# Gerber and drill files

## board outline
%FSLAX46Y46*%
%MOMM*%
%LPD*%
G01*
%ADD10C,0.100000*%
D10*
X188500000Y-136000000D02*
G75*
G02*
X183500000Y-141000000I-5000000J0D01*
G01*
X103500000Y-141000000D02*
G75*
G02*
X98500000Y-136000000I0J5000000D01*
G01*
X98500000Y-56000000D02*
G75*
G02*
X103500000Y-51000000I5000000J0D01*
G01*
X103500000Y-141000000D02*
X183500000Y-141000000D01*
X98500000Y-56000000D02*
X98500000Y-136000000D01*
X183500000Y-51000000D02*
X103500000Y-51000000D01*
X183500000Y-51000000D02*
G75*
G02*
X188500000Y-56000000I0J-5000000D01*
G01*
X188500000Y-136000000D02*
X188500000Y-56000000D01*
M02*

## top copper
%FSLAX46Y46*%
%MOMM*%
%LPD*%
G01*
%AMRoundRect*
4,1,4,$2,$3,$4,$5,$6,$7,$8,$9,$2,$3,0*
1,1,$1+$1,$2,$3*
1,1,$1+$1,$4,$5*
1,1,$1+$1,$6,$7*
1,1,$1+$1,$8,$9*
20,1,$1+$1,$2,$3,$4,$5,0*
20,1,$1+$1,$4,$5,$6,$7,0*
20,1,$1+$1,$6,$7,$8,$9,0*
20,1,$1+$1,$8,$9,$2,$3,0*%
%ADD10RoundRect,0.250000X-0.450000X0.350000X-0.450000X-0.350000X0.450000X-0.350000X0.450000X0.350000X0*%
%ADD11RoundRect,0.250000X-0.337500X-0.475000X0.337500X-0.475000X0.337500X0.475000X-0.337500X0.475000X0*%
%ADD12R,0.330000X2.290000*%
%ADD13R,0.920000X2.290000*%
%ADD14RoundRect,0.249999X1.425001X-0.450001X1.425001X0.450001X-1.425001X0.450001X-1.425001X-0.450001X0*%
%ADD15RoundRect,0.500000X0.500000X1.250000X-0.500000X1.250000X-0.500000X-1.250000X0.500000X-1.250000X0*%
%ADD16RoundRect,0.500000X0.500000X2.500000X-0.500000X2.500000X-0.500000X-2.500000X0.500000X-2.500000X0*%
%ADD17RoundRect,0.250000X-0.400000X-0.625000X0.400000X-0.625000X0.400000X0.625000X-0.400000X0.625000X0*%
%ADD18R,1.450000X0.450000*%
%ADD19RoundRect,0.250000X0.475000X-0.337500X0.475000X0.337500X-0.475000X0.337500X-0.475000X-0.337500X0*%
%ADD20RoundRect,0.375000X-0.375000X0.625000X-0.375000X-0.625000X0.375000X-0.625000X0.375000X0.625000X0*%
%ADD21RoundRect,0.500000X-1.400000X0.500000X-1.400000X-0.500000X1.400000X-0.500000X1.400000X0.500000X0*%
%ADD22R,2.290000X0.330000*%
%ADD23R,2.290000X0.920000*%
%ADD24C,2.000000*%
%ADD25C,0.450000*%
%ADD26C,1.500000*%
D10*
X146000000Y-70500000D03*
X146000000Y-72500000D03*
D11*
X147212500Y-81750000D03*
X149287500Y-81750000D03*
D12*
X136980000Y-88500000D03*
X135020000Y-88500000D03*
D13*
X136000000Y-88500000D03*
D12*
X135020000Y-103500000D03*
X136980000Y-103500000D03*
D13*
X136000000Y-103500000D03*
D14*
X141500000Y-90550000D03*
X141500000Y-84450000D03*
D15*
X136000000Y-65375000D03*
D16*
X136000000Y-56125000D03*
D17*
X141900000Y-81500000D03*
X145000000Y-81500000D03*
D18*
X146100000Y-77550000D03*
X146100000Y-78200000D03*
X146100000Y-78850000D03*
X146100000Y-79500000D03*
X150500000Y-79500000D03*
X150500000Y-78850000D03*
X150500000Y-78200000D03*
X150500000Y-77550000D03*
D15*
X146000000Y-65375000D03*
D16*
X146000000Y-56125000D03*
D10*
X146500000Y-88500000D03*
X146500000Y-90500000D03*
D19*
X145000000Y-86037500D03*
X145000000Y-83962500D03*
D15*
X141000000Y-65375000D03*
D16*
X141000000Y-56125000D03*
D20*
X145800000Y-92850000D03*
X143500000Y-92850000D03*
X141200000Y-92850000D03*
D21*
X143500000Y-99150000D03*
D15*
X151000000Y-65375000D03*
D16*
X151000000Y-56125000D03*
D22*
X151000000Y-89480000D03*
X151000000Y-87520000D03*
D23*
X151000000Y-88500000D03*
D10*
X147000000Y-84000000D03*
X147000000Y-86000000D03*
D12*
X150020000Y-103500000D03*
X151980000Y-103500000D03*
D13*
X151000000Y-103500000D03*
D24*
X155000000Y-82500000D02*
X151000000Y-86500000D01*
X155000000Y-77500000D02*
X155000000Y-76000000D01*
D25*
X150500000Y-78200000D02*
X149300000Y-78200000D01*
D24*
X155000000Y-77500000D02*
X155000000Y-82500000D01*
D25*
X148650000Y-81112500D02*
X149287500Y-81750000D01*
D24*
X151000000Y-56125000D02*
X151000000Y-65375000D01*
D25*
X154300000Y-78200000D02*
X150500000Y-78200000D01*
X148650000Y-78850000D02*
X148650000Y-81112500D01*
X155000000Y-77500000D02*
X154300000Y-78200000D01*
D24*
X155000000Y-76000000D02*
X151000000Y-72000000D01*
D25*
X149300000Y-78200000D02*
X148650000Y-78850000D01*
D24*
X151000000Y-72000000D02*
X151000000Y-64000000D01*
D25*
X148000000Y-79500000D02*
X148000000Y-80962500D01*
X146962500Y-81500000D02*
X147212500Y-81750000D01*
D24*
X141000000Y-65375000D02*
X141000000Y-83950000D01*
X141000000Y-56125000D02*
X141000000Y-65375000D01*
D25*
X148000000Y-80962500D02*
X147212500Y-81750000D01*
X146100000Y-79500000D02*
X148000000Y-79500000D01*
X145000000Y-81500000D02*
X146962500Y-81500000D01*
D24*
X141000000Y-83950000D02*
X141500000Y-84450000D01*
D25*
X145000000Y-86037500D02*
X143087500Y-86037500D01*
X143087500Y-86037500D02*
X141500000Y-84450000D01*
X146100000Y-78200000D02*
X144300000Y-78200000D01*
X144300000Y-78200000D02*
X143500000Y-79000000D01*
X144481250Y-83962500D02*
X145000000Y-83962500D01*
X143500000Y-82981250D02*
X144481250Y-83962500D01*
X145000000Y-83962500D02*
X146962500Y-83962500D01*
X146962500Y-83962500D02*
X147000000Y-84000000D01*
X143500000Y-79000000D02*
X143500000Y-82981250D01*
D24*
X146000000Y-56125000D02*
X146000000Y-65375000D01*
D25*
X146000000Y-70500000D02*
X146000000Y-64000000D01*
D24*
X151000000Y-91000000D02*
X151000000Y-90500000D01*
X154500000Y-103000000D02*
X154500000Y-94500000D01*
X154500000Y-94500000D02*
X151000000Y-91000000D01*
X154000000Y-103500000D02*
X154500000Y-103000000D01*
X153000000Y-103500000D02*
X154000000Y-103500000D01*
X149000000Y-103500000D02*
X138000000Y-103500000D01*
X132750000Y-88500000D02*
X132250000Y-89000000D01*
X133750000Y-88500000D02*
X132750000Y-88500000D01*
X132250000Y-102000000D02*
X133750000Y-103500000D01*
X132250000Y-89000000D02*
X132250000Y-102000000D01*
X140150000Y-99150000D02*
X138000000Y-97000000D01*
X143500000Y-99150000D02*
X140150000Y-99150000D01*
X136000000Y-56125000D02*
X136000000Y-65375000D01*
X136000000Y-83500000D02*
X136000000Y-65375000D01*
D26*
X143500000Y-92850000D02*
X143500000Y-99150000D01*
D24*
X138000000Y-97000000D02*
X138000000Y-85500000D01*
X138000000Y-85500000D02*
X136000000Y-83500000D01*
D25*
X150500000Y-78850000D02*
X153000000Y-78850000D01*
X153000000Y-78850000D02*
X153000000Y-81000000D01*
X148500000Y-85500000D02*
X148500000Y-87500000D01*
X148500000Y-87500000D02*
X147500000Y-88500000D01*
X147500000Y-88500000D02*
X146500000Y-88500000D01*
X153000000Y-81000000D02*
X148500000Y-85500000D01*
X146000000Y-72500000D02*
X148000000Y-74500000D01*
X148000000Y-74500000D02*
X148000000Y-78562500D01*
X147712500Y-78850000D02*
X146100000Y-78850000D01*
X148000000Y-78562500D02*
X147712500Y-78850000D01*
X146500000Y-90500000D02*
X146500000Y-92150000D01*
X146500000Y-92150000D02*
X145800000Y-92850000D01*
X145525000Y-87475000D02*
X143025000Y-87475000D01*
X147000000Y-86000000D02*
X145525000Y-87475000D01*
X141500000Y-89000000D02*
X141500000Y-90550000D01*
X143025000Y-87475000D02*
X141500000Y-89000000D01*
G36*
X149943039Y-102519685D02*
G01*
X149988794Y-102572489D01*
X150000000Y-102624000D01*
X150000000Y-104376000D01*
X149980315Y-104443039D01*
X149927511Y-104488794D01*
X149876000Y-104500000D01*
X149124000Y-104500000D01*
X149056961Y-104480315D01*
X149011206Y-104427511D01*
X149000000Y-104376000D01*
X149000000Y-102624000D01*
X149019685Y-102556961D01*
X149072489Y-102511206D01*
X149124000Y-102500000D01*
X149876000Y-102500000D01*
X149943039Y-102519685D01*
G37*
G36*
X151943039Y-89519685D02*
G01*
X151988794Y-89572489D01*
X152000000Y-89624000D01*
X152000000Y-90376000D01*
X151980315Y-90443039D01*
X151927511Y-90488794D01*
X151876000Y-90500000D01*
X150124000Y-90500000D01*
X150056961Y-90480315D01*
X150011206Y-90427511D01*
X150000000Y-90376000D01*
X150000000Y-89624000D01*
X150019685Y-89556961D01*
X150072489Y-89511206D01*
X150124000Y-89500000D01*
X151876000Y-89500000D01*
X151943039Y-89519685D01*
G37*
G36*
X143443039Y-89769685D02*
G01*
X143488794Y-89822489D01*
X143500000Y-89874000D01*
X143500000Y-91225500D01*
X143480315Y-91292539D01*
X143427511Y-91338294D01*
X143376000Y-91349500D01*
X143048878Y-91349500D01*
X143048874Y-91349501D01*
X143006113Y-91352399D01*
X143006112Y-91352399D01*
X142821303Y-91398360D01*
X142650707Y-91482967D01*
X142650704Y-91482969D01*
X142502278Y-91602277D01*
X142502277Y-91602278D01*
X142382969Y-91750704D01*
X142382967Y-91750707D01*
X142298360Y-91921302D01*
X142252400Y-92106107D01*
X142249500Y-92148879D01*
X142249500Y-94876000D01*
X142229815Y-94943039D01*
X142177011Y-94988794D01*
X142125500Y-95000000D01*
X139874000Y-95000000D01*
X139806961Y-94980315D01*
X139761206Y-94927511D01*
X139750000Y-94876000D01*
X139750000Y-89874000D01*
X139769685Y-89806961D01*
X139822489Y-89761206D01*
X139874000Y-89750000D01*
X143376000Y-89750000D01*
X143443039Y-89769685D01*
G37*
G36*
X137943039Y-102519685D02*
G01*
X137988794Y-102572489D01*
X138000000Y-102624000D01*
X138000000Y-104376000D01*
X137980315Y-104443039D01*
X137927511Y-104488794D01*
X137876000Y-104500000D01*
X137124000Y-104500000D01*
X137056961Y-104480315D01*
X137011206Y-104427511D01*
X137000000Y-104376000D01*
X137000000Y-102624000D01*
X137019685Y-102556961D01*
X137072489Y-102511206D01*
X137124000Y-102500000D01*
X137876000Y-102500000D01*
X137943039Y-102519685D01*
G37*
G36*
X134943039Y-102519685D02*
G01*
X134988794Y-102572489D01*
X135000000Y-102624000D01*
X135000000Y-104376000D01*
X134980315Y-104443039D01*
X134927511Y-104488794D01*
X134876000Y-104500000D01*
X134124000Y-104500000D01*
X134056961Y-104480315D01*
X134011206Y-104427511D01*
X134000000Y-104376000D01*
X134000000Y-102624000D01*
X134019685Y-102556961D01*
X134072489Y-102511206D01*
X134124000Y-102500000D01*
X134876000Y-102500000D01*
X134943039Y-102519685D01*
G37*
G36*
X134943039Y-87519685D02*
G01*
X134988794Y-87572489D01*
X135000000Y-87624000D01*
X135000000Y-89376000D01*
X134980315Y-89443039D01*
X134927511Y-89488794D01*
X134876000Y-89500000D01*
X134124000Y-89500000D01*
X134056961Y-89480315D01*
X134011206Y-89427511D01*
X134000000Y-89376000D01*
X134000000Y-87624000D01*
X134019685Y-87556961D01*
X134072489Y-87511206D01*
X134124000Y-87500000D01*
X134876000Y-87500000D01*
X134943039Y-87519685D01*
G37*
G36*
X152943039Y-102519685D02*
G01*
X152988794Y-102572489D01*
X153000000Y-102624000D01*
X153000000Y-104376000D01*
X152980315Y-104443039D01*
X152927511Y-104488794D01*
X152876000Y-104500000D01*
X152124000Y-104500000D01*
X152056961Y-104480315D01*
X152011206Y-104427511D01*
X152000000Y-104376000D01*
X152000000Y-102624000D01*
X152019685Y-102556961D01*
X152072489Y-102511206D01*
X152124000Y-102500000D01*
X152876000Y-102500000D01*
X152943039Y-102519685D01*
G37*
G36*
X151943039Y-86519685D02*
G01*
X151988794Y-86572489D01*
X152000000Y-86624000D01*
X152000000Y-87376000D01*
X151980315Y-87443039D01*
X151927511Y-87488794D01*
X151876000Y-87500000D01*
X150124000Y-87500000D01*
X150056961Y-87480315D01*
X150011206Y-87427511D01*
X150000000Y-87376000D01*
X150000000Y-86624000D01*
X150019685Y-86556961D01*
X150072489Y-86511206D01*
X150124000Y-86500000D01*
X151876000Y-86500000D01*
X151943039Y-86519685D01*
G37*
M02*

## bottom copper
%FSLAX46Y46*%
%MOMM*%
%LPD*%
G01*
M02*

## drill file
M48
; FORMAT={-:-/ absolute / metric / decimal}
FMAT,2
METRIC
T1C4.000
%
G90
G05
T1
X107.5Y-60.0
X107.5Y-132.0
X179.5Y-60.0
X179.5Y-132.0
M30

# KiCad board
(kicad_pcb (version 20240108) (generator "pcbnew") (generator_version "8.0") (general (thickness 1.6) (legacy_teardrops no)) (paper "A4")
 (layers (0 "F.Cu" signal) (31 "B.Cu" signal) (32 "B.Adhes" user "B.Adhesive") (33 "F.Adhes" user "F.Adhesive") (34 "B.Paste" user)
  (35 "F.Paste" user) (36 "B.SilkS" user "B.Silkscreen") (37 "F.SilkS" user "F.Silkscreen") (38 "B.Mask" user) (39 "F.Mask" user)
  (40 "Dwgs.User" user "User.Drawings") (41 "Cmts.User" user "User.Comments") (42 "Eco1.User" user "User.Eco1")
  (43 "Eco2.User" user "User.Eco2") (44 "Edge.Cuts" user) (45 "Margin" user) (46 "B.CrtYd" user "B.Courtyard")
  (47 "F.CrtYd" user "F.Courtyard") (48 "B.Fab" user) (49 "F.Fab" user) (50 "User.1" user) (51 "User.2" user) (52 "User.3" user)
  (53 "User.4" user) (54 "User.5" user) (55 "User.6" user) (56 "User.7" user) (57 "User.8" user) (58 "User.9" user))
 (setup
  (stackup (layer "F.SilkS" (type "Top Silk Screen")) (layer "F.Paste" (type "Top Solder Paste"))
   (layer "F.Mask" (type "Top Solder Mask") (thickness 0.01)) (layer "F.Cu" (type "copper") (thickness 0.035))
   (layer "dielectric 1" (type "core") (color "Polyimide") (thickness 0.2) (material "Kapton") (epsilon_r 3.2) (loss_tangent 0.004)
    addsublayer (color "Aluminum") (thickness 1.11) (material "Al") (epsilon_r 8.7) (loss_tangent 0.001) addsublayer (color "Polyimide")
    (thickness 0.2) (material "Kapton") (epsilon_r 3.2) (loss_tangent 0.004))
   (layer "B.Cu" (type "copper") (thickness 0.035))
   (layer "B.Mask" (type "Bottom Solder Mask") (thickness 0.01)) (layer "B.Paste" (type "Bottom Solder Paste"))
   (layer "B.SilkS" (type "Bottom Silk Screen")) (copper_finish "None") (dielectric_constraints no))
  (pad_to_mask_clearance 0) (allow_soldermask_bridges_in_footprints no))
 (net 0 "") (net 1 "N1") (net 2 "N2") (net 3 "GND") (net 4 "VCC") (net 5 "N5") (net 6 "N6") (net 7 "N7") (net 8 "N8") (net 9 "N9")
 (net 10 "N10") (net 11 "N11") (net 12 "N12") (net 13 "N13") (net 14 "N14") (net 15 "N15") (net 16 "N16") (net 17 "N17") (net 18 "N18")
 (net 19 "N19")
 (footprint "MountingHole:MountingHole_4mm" (layer "F.Cu") (at 179.5 132)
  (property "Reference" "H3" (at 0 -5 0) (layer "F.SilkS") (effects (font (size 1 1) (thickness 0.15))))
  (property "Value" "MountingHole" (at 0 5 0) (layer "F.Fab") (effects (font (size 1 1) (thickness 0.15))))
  (pad "" np_thru_hole circle (at 0 0) (size 4 4) (drill 4) (layers "*.Cu" "*.Mask")))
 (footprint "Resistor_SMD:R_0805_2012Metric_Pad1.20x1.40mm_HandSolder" (layer "F.Cu") (at 146 71.5 -90)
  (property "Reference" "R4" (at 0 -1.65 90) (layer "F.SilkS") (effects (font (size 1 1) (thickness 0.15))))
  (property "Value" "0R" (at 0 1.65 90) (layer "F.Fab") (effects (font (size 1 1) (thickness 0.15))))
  (pad "1" smd roundrect (at -1 0 270) (size 1.2 1.4) (layers "F.Cu" "F.Paste" "F.Mask") (roundrect_rratio 0.208333) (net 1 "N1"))
  (pad "2" smd roundrect (at 1 0 270) (size 1.2 1.4) (layers "F.Cu" "F.Paste" "F.Mask") (roundrect_rratio 0.208333) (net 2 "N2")))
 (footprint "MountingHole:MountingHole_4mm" (layer "F.Cu") (at 107.5 60)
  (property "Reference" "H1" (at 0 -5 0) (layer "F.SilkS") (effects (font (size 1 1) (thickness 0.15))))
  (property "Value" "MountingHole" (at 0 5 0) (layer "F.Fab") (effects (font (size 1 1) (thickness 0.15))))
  (pad "" np_thru_hole circle (at 0 0) (size 4 4) (drill 4) (layers "*.Cu" "*.Mask")))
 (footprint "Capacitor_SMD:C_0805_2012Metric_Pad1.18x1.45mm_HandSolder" (layer "F.Cu") (at 148.25 81.75)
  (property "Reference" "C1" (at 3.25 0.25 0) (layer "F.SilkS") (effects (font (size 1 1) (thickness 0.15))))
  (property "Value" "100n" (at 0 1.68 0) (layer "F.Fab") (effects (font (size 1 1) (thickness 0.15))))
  (pad "1" smd roundrect (at -1.0375 0) (size 1.175 1.45) (layers "F.Cu" "F.Paste" "F.Mask") (roundrect_rratio 0.212766) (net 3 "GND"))
  (pad "2" smd roundrect (at 1.0375 0) (size 1.175 1.45) (layers "F.Cu" "F.Paste" "F.Mask") (roundrect_rratio 0.212766) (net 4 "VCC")))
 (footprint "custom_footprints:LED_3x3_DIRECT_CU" (layer "F.Cu") (at 136 88.5 180)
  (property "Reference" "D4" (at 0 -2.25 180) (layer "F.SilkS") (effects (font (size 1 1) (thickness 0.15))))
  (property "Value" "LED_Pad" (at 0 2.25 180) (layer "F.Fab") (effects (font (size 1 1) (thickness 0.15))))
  (pad "" smd rect (at 0 -0.55 180) (size 0.85 0.85) (layers "F.Paste"))
  (pad "" smd rect (at 0 0 180) (size 0.92 2.29) (layers "Eco1.User"))
  (pad "" smd rect (at 0 0.55 180) (size 0.85 0.85) (layers "F.Paste"))
  (pad "1" smd rect (at -0.98 0 180) (size 0.33 2.29) (layers "F.Cu" "F.Paste" "F.Mask") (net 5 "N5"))
  (pad "2" smd rect (at 0.98 0 180) (size 0.33 2.29) (layers "F.Cu" "F.Paste" "F.Mask") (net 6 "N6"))
  (pad "3" smd rect (at 0 0 180) (size 0.92 2.29) (layers "F.Cu" "F.Mask") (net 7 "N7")))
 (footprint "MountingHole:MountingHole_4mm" (layer "F.Cu") (at 107.5 132)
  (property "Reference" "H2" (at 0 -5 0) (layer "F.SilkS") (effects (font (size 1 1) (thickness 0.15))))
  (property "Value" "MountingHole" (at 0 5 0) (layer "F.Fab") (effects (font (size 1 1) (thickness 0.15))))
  (pad "" np_thru_hole circle (at 0 0) (size 4 4) (drill 4) (layers "*.Cu" "*.Mask")))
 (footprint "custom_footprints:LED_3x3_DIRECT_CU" (layer "F.Cu") (at 136 103.5)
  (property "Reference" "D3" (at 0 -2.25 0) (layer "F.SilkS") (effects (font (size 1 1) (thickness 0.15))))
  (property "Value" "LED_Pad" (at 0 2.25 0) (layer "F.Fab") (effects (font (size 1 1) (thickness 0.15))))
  (pad "" smd rect (at 0 -0.55) (size 0.85 0.85) (layers "F.Paste"))
  (pad "" smd rect (at 0 0) (size 0.92 2.29) (layers "Eco1.User"))
  (pad "" smd rect (at 0 0.55) (size 0.85 0.85) (layers "F.Paste"))
  (pad "1" smd rect (at -0.98 0) (size 0.33 2.29) (layers "F.Cu" "F.Paste" "F.Mask") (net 6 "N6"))
  (pad "2" smd rect (at 0.98 0) (size 0.33 2.29) (layers "F.Cu" "F.Paste" "F.Mask") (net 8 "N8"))
  (pad "3" smd rect (at 0 0) (size 0.92 2.29) (layers "F.Cu" "F.Mask") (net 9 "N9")))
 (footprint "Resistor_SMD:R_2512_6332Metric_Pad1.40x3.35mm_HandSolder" (layer "F.Cu") (at 141.5 87.5 90)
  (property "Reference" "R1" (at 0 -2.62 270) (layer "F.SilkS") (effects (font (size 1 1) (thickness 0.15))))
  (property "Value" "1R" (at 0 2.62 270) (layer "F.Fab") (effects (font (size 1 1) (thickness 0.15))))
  (pad "1" smd roundrect (at -3.05 0 90) (size 1.4 3.35) (layers "F.Cu" "F.Paste" "F.Mask") (roundrect_rratio 0.178571) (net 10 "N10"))
  (pad "2" smd roundrect (at 3.05 0 90) (size 1.4 3.35) (layers "F.Cu" "F.Paste" "F.Mask") (roundrect_rratio 0.178571) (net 3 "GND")))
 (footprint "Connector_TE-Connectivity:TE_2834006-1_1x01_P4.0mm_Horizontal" (layer "F.Cu") (at 136 60.125 180)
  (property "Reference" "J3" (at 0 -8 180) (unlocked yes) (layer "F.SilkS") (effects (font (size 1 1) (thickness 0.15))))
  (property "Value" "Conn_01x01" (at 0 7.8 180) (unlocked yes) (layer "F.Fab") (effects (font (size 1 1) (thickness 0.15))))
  (pad "1" smd roundrect (at 0 -5.25 180) (size 2 3.5) (layers "F.Cu" "F.Paste" "F.Mask") (roundrect_rratio 0.25) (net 5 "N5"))
  (pad "1" smd roundrect (at 0 4 180) (size 2 6) (layers "F.Cu" "F.Paste" "F.Mask") (roundrect_rratio 0.25) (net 5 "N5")))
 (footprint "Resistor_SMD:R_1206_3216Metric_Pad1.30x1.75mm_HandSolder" (layer "F.Cu") (at 143.45 81.5)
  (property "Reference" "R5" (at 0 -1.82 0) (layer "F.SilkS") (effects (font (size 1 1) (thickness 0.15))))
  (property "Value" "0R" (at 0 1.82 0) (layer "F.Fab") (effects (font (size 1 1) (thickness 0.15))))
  (pad "1" smd roundrect (at -1.55 0) (size 1.3 1.75) (layers "F.Cu" "F.Paste" "F.Mask") (roundrect_rratio 0.192308) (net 3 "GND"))
  (pad "2" smd roundrect (at 1.55 0) (size 1.3 1.75) (layers "F.Cu" "F.Paste" "F.Mask") (roundrect_rratio 0.192308) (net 3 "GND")))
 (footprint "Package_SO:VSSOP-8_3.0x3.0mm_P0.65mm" (layer "F.Cu") (at 148.3 78.525)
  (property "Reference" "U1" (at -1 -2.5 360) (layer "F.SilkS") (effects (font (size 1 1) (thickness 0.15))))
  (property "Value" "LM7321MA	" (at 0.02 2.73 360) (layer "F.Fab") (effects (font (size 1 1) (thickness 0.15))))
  (pad "1" smd rect (at -2.2 -0.975 270) (size 0.45 1.45) (layers "F.Cu" "F.Paste" "F.Mask") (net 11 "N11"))
  (pad "2" smd rect (at -2.2 -0.325 270) (size 0.45 1.45) (layers "F.Cu" "F.Paste" "F.Mask") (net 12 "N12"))
  (pad "3" smd rect (at -2.2 0.325 270) (size 0.45 1.45) (layers "F.Cu" "F.Paste" "F.Mask") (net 2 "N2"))
  (pad "4" smd rect (at -2.2 0.975 270) (size 0.45 1.45) (layers "F.Cu" "F.Paste" "F.Mask") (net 3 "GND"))
  (pad "5" smd rect (at 2.2 0.975 270) (size 0.45 1.45) (layers "F.Cu" "F.Paste" "F.Mask") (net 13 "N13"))
  (pad "6" smd rect (at 2.2 0.325 270) (size 0.45 1.45) (layers "F.Cu" "F.Paste" "F.Mask") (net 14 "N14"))
  (pad "7" smd rect (at 2.2 -0.325 270) (size 0.45 1.45) (layers "F.Cu" "F.Paste" "F.Mask") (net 4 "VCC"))
  (pad "8" smd rect (at 2.2 -0.975 270) (size 0.45 1.45) (layers "F.Cu" "F.Paste" "F.Mask") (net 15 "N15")))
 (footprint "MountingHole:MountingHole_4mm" (layer "F.Cu") (at 179.5 60)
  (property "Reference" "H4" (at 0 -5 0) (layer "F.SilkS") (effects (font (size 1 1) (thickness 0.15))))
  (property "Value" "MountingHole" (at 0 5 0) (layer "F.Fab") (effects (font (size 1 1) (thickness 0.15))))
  (pad "" np_thru_hole circle (at 0 0) (size 4 4) (drill 4) (layers "*.Cu" "*.Mask")))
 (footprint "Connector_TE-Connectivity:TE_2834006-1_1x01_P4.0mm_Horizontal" (layer "F.Cu") (at 146 60.125 180)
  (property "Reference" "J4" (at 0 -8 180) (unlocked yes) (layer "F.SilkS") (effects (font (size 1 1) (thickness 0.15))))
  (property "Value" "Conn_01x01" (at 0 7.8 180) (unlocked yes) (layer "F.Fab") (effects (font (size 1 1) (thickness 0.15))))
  (pad "1" smd roundrect (at 0 -5.25 180) (size 2 3.5) (layers "F.Cu" "F.Paste" "F.Mask") (roundrect_rratio 0.25) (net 1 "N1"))
  (pad "1" smd roundrect (at 0 4 180) (size 2 6) (layers "F.Cu" "F.Paste" "F.Mask") (roundrect_rratio 0.25) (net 1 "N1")))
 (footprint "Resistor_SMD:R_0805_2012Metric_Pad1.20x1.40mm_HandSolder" (layer "F.Cu") (at 146.5 89.5 -90)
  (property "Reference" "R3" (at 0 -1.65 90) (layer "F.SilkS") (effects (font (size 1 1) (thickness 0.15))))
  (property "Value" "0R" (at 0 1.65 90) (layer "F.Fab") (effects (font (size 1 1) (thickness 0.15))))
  (pad "1" smd roundrect (at -1 0 270) (size 1.2 1.4) (layers "F.Cu" "F.Paste" "F.Mask") (roundrect_rratio 0.208333) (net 14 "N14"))
  (pad "2" smd roundrect (at 1 0 270) (size 1.2 1.4) (layers "F.Cu" "F.Paste" "F.Mask") (roundrect_rratio 0.208333) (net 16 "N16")))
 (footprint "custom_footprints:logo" (layer "F.Cu") (at 144 138.5)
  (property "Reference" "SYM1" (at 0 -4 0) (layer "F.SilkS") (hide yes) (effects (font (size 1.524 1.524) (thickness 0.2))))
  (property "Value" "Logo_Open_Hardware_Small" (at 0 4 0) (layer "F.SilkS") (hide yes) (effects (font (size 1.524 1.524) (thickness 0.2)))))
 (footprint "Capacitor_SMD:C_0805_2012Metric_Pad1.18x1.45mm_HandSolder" (layer "F.Cu") (at 145 85 90)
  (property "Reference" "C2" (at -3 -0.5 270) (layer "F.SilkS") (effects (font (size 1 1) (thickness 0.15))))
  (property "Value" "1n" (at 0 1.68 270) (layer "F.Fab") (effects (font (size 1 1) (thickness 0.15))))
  (pad "1" smd roundrect (at -1.0375 0 90) (size 1.175 1.45) (layers "F.Cu" "F.Paste" "F.Mask") (roundrect_rratio 0.212766) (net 3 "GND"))
  (pad "2" smd roundrect (at 1.0375 0 90) (size 1.175 1.45) (layers "F.Cu" "F.Paste" "F.Mask") (roundrect_rratio 0.212766) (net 12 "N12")))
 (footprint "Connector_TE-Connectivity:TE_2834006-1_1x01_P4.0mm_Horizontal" (layer "F.Cu") (at 141 60.125 180)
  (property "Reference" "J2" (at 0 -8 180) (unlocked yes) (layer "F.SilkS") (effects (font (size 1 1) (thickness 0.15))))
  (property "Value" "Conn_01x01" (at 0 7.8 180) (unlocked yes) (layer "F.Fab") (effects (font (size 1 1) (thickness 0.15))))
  (pad "1" smd roundrect (at 0 -5.25 180) (size 2 3.5) (layers "F.Cu" "F.Paste" "F.Mask") (roundrect_rratio 0.25) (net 3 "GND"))
  (pad "1" smd roundrect (at 0 4 180) (size 2 6) (layers "F.Cu" "F.Paste" "F.Mask") (roundrect_rratio 0.25) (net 3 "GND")))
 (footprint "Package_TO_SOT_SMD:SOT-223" (layer "F.Cu") (at 143.5 96 -90)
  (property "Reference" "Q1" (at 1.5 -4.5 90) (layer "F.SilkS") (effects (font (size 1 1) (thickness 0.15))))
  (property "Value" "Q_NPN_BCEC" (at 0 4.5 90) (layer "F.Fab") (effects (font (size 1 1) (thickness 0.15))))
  (pad "1" smd roundrect (at -3.15 -2.3 270) (size 2 1.5) (layers "F.Cu" "F.Paste" "F.Mask") (roundrect_rratio 0.25) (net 16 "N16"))
  (pad "2" smd roundrect (at -3.15 0 270) (size 2 1.5) (layers "F.Cu" "F.Paste" "F.Mask") (roundrect_rratio 0.25) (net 5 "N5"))
  (pad "3" smd roundrect (at -3.15 2.3 270) (size 2 1.5) (layers "F.Cu" "F.Paste" "F.Mask") (roundrect_rratio 0.25) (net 10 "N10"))
  (pad "4" smd roundrect (at 3.15 0 270) (size 2 3.8) (layers "F.Cu" "F.Paste" "F.Mask") (roundrect_rratio 0.25) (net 5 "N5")))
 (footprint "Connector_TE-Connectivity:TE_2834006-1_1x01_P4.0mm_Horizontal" (layer "F.Cu") (at 151 60.125 180)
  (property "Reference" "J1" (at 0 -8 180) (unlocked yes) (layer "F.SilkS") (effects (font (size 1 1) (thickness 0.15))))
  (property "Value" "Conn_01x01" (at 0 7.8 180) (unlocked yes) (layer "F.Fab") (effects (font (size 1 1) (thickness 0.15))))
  (pad "1" smd roundrect (at 0 -5.25 180) (size 2 3.5) (layers "F.Cu" "F.Paste" "F.Mask") (roundrect_rratio 0.25) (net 4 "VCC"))
  (pad "1" smd roundrect (at 0 4 180) (size 2 6) (layers "F.Cu" "F.Paste" "F.Mask") (roundrect_rratio 0.25) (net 4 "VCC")))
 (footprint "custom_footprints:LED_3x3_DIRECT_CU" (layer "F.Cu") (at 151 88.5 90)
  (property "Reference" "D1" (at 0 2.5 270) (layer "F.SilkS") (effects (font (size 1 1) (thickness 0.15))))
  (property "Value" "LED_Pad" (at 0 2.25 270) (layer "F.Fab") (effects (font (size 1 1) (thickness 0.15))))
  (pad "" smd rect (at 0 -0.55 90) (size 0.85 0.85) (layers "F.Paste"))
  (pad "" smd rect (at 0 0 90) (size 0.92 2.29) (layers "Eco1.User"))
  (pad "" smd rect (at 0 0.55 90) (size 0.85 0.85) (layers "F.Paste"))
  (pad "1" smd rect (at -0.98 0 90) (size 0.33 2.29) (layers "F.Cu" "F.Paste" "F.Mask") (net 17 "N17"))
  (pad "2" smd rect (at 0.98 0 90) (size 0.33 2.29) (layers "F.Cu" "F.Paste" "F.Mask") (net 4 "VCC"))
  (pad "3" smd rect (at 0 0 90) (size 0.92 2.29) (layers "F.Cu" "F.Mask") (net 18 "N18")))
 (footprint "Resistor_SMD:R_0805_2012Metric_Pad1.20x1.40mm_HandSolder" (layer "F.Cu") (at 147 85 -90)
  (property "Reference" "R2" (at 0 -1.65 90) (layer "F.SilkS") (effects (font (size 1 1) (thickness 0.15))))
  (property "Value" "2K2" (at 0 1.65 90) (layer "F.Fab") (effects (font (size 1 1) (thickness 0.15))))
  (pad "1" smd roundrect (at -1 0 270) (size 1.2 1.4) (layers "F.Cu" "F.Paste" "F.Mask") (roundrect_rratio 0.208333) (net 12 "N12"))
  (pad "2" smd roundrect (at 1 0 270) (size 1.2 1.4) (layers "F.Cu" "F.Paste" "F.Mask") (roundrect_rratio 0.208333) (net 10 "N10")))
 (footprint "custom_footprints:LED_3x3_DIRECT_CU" (layer "F.Cu") (at 151 103.5)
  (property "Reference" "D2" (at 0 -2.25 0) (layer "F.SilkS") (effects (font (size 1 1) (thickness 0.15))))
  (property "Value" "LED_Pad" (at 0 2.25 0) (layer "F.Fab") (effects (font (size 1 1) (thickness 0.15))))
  (pad "" smd rect (at 0 -0.55) (size 0.85 0.85) (layers "F.Paste"))
  (pad "" smd rect (at 0 0) (size 0.92 2.29) (layers "Eco1.User"))
  (pad "" smd rect (at 0 0.55) (size 0.85 0.85) (layers "F.Paste"))
  (pad "1" smd rect (at -0.98 0) (size 0.33 2.29) (layers "F.Cu" "F.Paste" "F.Mask") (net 8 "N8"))
  (pad "2" smd rect (at 0.98 0) (size 0.33 2.29) (layers "F.Cu" "F.Paste" "F.Mask") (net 17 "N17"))
  (pad "3" smd rect (at 0 0) (size 0.92 2.29) (layers "F.Cu" "F.Mask") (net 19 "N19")))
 (gr_arc (start 188.5 136) (mid 187.035534 139.535534) (end 183.5 141) (stroke (width 0.1) (type default)) (layer "Edge.Cuts"))
 (gr_arc (start 103.5 141) (mid 99.964466 139.535534) (end 98.5 136) (stroke (width 0.1) (type default)) (layer "Edge.Cuts"))
 (gr_arc (start 98.5 56) (mid 99.964466 52.464466) (end 103.5 51) (stroke (width 0.1) (type default)) (layer "Edge.Cuts"))
 (gr_line (start 103.5 141) (end 183.5 141) (stroke (width 0.1) (type default)) (layer "Edge.Cuts"))
 (gr_line (start 98.5 56) (end 98.5 136) (stroke (width 0.1) (type default)) (layer "Edge.Cuts"))
 (gr_line (start 183.5 51) (end 103.5 51) (stroke (width 0.1) (type default)) (layer "Edge.Cuts"))
 (gr_arc (start 183.5 51) (mid 187.035534 52.464466) (end 188.5 56) (stroke (width 0.1) (type default)) (layer "Edge.Cuts"))
 (gr_line (start 188.5 136) (end 188.5 56) (stroke (width 0.1) (type default)) (layer "Edge.Cuts"))
 (segment (start 155 82.5) (end 151 86.5) (width 2) (layer "F.Cu") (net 4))
 (segment (start 155 77.5) (end 155 76) (width 2) (layer "F.Cu") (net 4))
 (segment (start 150.5 78.2) (end 149.3 78.2) (width 0.45) (layer "F.Cu") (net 4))
 (segment (start 155 77.5) (end 155 82.5) (width 2) (layer "F.Cu") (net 4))
 (segment (start 148.65 81.1125) (end 149.2875 81.75) (width 0.45) (layer "F.Cu") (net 4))
 (segment (start 151 56.125) (end 151 65.375) (width 2) (layer "F.Cu") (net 4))
 (segment (start 154.3 78.2) (end 150.5 78.2) (width 0.45) (layer "F.Cu") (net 4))
 (segment (start 148.65 78.85) (end 148.65 81.1125) (width 0.45) (layer "F.Cu") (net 4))
 (segment (start 155 77.5) (end 154.3 78.2) (width 0.45) (layer "F.Cu") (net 4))
 (segment (start 155 76) (end 151 72) (width 2) (layer "F.Cu") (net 4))
 (segment (start 149.3 78.2) (end 148.65 78.85) (width 0.45) (layer "F.Cu") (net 4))
 (segment (start 151 72) (end 151 64) (width 2) (layer "F.Cu") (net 4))
 (segment (start 148 79.5) (end 148 80.9625) (width 0.45) (layer "F.Cu") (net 3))
 (segment (start 146.9625 81.5) (end 147.2125 81.75) (width 0.45) (layer "F.Cu") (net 3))
 (segment (start 141 65.375) (end 141 83.95) (width 2) (layer "F.Cu") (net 3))
 (segment (start 141 56.125) (end 141 65.375) (width 2) (layer "F.Cu") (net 3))
 (segment (start 148 80.9625) (end 147.2125 81.75) (width 0.45) (layer "F.Cu") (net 3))
 (segment (start 146.1 79.5) (end 148 79.5) (width 0.45) (layer "F.Cu") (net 3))
 (segment (start 145 81.5) (end 146.9625 81.5) (width 0.45) (layer "F.Cu") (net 3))
 (segment (start 141 83.95) (end 141.5 84.45) (width 2) (layer "F.Cu") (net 3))
 (segment (start 145 86.0375) (end 143.0875 86.0375) (width 0.45) (layer "F.Cu") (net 3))
 (segment (start 143.0875 86.0375) (end 141.5 84.45) (width 0.45) (layer "F.Cu") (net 3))
 (segment (start 146.1 78.2) (end 144.3 78.2) (width 0.45) (layer "F.Cu") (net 12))
 (segment (start 144.3 78.2) (end 143.5 79) (width 0.45) (layer "F.Cu") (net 12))
 (segment (start 144.48125 83.9625) (end 145 83.9625) (width 0.45) (layer "F.Cu") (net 12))
 (segment (start 143.5 82.98125) (end 144.48125 83.9625) (width 0.45) (layer "F.Cu") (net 12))
 (segment (start 145 83.9625) (end 146.9625 83.9625) (width 0.45) (layer "F.Cu") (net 12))
 (segment (start 146.9625 83.9625) (end 147 84) (width 0.45) (layer "F.Cu") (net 12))
 (segment (start 143.5 79) (end 143.5 82.98125) (width 0.45) (layer "F.Cu") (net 12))
 (segment (start 146 56.125) (end 146 65.375) (width 2) (layer "F.Cu") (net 1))
 (segment (start 146 70.5) (end 146 64) (width 0.45) (layer "F.Cu") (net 1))
 (segment (start 151 91) (end 151 90.5) (width 2) (layer "F.Cu") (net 17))
 (segment (start 154.5 103) (end 154.5 94.5) (width 2) (layer "F.Cu") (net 17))
 (segment (start 154.5 94.5) (end 151 91) (width 2) (layer "F.Cu") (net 17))
 (segment (start 154 103.5) (end 154.5 103) (width 2) (layer "F.Cu") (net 17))
 (segment (start 153 103.5) (end 154 103.5) (width 2) (layer "F.Cu") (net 17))
 (segment (start 149 103.5) (end 138 103.5) (width 2) (layer "F.Cu") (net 8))
 (segment (start 132.75 88.5) (end 132.25 89) (width 2) (layer "F.Cu") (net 6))
 (segment (start 133.75 88.5) (end 132.75 88.5) (width 2) (layer "F.Cu") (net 6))
 (segment (start 132.25 102) (end 133.75 103.5) (width 2) (layer "F.Cu") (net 6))
 (segment (start 132.25 89) (end 132.25 102) (width 2) (layer "F.Cu") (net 6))
 (segment (start 140.15 99.15) (end 138 97) (width 2) (layer "F.Cu") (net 5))
 (segment (start 143.5 99.15) (end 140.15 99.15) (width 2) (layer "F.Cu") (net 5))
 (segment (start 136 56.125) (end 136 65.375) (width 2) (layer "F.Cu") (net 5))
 (segment (start 136 83.5) (end 136 65.375) (width 2) (layer "F.Cu") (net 5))
 (segment (start 143.5 92.85) (end 143.5 99.15) (width 1.5) (layer "F.Cu") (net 5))
 (segment (start 138 97) (end 138 85.5) (width 2) (layer "F.Cu") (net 5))
 (segment (start 138 85.5) (end 136 83.5) (width 2) (layer "F.Cu") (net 5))
 (segment (start 150.5 78.85) (end 153 78.85) (width 0.45) (layer "F.Cu") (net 14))
 (segment (start 153 78.85) (end 153 81) (width 0.45) (layer "F.Cu") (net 14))
 (segment (start 148.5 85.5) (end 148.5 87.5) (width 0.45) (layer "F.Cu") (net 14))
 (segment (start 148.5 87.5) (end 147.5 88.5) (width 0.45) (layer "F.Cu") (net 14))
 (segment (start 147.5 88.5) (end 146.5 88.5) (width 0.45) (layer "F.Cu") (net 14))
 (segment (start 153 81) (end 148.5 85.5) (width 0.45) (layer "F.Cu") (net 14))
 (segment (start 146 72.5) (end 148 74.5) (width 0.45) (layer "F.Cu") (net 2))
 (segment (start 148 74.5) (end 148 78.5625) (width 0.45) (layer "F.Cu") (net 2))
 (segment (start 147.7125 78.85) (end 146.1 78.85) (width 0.45) (layer "F.Cu") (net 2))
 (segment (start 148 78.5625) (end 147.7125 78.85) (width 0.45) (layer "F.Cu") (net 2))
 (segment (start 146.5 90.5) (end 146.5 92.15) (width 0.45) (layer "F.Cu") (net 16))
 (segment (start 146.5 92.15) (end 145.8 92.85) (width 0.45) (layer "F.Cu") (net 16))
 (segment (start 145.525 87.475) (end 143.025 87.475) (width 0.45) (layer "F.Cu") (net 10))
 (segment (start 147 86) (end 145.525 87.475) (width 0.45) (layer "F.Cu") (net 10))
 (segment (start 141.5 89) (end 141.5 90.55) (width 0.45) (layer "F.Cu") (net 10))
 (segment (start 143.025 87.475) (end 141.5 89) (width 0.45) (layer "F.Cu") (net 10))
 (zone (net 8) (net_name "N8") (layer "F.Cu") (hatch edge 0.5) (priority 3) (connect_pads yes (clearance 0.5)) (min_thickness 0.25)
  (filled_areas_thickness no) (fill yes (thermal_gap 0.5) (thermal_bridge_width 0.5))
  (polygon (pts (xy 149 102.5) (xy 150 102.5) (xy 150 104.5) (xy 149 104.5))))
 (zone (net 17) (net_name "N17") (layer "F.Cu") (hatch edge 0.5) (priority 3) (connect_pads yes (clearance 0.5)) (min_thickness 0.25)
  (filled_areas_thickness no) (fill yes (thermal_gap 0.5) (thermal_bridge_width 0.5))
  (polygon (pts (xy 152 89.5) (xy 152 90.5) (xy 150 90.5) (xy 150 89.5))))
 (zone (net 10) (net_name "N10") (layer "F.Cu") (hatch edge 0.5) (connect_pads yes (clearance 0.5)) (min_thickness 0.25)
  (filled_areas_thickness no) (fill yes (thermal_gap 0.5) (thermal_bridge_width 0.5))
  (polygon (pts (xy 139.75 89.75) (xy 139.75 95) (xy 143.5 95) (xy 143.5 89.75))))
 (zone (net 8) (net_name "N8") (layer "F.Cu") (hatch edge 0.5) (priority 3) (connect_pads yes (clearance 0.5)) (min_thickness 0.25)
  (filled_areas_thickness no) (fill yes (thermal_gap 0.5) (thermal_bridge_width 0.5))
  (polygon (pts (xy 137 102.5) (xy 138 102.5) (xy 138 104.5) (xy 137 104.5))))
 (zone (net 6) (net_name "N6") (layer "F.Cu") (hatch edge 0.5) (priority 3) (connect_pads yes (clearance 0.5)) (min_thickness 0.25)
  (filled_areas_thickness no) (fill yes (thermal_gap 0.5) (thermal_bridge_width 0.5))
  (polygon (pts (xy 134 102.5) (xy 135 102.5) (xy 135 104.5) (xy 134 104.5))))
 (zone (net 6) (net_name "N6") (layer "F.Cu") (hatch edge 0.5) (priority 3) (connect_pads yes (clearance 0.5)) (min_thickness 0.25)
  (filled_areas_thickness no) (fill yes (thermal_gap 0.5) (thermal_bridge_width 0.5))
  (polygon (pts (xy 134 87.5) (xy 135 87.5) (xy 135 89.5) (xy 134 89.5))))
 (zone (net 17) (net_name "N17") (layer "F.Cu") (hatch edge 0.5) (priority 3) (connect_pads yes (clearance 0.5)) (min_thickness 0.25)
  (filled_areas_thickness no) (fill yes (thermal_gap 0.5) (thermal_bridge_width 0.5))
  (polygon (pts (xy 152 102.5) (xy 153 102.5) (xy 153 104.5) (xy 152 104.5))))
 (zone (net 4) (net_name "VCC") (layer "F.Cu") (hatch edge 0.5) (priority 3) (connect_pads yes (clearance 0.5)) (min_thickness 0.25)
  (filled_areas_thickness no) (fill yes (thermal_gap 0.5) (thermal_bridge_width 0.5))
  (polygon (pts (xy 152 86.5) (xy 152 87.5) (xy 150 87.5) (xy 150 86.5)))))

